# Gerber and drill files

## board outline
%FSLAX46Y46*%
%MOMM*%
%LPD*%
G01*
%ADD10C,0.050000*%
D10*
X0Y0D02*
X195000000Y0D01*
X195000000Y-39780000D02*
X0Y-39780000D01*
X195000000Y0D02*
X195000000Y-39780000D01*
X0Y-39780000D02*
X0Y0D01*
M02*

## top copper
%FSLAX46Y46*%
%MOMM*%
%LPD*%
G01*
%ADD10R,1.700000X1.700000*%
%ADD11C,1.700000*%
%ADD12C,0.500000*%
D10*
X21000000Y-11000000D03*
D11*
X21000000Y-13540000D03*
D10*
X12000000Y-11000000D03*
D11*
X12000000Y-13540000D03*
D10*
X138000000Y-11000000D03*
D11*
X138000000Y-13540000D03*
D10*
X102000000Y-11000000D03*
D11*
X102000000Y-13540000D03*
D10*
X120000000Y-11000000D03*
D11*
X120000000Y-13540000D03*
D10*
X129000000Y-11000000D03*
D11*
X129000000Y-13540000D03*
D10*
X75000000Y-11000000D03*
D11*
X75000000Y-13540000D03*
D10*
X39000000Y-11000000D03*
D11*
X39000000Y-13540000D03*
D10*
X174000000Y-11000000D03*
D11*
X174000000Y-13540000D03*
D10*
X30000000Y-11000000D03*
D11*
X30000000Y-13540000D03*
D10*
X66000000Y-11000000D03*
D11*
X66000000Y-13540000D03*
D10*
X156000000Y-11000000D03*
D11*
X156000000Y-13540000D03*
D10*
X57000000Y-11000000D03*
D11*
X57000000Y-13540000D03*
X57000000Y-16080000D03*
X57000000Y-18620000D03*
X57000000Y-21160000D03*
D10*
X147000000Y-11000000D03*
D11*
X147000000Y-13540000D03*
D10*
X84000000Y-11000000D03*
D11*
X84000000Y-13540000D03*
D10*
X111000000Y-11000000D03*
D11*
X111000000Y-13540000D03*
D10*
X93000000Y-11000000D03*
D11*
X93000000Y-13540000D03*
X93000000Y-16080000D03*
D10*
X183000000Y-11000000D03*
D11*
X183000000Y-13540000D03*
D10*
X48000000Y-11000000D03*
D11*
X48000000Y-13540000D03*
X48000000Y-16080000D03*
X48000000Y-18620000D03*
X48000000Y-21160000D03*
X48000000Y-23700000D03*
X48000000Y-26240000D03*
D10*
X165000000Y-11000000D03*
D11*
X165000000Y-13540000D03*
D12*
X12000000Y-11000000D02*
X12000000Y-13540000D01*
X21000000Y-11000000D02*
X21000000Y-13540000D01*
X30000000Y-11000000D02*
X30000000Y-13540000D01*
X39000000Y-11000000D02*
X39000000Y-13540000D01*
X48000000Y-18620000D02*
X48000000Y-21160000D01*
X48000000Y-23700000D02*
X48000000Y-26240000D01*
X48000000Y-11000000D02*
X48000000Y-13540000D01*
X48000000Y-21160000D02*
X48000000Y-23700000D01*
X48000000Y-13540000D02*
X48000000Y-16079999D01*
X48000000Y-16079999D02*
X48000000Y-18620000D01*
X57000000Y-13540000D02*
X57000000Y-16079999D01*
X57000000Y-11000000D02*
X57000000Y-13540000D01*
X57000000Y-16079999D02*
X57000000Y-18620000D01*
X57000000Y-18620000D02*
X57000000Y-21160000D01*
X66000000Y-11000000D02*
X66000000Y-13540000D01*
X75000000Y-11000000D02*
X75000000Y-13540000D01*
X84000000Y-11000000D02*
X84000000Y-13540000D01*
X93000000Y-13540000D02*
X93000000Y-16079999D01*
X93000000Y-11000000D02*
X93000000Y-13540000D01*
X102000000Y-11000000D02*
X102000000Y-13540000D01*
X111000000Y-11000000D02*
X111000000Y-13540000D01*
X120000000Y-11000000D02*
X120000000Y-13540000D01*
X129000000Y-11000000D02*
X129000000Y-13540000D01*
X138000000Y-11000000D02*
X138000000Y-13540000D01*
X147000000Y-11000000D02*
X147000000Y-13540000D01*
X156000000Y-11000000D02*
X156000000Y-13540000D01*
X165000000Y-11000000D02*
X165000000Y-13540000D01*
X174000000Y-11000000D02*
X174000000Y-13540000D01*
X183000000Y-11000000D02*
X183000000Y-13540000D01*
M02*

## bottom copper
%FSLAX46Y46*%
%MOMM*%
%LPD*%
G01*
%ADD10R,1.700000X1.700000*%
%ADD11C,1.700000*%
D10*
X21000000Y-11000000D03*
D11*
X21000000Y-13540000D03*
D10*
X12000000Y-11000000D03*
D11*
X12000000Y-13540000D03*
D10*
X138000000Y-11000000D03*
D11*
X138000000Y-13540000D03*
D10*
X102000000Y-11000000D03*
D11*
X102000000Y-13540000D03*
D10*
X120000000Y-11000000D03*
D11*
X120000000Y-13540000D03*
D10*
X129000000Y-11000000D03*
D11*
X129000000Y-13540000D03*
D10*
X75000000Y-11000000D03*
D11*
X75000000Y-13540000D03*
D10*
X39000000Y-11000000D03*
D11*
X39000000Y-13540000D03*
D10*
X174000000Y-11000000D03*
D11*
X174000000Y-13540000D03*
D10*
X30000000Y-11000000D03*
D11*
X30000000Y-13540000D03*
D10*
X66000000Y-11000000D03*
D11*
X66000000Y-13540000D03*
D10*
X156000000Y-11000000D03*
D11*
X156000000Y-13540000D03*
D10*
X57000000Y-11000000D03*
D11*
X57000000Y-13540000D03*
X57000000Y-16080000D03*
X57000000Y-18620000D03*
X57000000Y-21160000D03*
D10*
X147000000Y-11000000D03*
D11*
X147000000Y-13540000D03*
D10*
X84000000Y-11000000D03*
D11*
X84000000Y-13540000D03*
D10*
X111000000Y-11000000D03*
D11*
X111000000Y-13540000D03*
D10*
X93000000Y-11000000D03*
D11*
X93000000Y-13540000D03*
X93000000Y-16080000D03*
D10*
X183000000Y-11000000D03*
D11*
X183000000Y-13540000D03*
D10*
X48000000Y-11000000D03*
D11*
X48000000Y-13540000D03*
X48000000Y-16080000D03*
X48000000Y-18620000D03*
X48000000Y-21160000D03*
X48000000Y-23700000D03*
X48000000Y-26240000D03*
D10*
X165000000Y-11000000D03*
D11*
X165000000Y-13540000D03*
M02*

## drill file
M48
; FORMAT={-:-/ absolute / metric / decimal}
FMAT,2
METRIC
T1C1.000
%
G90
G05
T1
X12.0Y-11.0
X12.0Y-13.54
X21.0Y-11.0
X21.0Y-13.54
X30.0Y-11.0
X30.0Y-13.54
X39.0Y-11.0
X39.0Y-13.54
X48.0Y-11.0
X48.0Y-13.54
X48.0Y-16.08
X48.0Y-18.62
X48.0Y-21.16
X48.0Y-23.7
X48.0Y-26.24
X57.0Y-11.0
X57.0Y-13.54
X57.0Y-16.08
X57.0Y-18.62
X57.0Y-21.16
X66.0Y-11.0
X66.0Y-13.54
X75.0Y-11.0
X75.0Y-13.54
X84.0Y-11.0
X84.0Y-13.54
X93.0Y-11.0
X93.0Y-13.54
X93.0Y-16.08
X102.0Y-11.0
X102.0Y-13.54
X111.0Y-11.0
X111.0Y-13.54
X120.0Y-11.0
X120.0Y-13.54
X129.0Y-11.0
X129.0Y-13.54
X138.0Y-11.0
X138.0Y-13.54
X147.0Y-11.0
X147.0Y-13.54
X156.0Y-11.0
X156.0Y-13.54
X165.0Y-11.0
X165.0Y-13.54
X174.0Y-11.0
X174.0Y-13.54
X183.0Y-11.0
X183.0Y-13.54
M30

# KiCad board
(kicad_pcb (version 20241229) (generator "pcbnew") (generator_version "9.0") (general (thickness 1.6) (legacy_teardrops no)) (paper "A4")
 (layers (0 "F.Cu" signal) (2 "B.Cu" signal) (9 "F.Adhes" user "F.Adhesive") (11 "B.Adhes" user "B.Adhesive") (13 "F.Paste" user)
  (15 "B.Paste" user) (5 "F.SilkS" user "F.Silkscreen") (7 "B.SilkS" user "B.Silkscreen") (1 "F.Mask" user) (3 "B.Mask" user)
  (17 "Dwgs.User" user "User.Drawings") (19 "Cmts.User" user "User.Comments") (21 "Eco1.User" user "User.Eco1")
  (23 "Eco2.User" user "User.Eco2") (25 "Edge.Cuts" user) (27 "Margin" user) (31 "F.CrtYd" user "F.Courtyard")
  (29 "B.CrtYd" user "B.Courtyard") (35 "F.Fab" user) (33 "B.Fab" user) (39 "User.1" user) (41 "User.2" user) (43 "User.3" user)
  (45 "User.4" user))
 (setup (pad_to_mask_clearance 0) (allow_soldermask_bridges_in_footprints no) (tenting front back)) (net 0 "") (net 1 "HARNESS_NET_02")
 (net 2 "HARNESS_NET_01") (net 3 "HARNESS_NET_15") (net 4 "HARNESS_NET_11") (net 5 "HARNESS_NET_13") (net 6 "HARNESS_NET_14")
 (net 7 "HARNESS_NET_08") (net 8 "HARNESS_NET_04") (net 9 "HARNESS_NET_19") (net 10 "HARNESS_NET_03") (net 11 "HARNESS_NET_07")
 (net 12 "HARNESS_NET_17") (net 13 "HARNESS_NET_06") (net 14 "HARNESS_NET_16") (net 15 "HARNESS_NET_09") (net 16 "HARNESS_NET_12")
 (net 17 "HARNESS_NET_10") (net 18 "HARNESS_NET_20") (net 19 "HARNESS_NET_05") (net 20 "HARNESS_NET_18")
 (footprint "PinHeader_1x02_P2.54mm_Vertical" (layer "F.Cu") (at 21 11)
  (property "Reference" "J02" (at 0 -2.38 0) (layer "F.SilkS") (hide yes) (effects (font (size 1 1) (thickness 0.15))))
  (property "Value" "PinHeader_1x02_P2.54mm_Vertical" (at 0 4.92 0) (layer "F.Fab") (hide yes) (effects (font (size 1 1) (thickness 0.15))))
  (pad "1" thru_hole rect (at 0 0) (size 1.7 1.7) (drill 1) (layers "*.Cu" "*.Mask") (remove_unused_layers no) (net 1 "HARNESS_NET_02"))
  (pad "2" thru_hole circle (at 0 2.54) (size 1.7 1.7) (drill 1) (layers "*.Cu" "*.Mask") (remove_unused_layers no) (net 1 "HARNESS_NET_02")))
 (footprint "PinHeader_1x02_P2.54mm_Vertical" (layer "F.Cu") (at 12 11)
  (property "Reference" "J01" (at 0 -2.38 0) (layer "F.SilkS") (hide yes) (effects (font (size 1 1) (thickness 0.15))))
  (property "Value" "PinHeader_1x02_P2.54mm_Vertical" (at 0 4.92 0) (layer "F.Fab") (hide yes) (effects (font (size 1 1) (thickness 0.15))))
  (pad "1" thru_hole rect (at 0 0) (size 1.7 1.7) (drill 1) (layers "*.Cu" "*.Mask") (remove_unused_layers no) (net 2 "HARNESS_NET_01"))
  (pad "2" thru_hole circle (at 0 2.54) (size 1.7 1.7) (drill 1) (layers "*.Cu" "*.Mask") (remove_unused_layers no) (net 2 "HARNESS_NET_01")))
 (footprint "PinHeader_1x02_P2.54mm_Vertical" (layer "F.Cu") (at 138 11)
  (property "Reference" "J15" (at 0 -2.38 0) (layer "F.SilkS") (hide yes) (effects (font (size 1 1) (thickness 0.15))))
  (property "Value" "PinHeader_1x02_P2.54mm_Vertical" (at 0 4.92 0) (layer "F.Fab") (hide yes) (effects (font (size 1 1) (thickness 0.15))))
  (pad "1" thru_hole rect (at 0 0) (size 1.7 1.7) (drill 1) (layers "*.Cu" "*.Mask") (remove_unused_layers no) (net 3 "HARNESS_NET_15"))
  (pad "2" thru_hole circle (at 0 2.54) (size 1.7 1.7) (drill 1) (layers "*.Cu" "*.Mask") (remove_unused_layers no) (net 3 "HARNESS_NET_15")))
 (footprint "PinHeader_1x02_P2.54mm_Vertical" (layer "F.Cu") (at 102 11)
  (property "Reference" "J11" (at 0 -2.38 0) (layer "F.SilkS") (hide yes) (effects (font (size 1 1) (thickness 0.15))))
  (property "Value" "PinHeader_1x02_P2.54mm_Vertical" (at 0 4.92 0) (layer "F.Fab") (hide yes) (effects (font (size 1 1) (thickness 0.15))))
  (pad "1" thru_hole rect (at 0 0) (size 1.7 1.7) (drill 1) (layers "*.Cu" "*.Mask") (remove_unused_layers no) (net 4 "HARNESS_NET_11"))
  (pad "2" thru_hole circle (at 0 2.54) (size 1.7 1.7) (drill 1) (layers "*.Cu" "*.Mask") (remove_unused_layers no) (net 4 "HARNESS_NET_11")))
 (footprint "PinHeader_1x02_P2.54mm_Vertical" (layer "F.Cu") (at 120 11)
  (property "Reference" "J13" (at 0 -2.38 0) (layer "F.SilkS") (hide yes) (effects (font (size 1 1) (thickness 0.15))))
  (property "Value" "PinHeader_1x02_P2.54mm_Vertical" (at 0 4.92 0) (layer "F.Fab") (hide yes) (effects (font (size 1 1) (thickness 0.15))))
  (pad "1" thru_hole rect (at 0 0) (size 1.7 1.7) (drill 1) (layers "*.Cu" "*.Mask") (remove_unused_layers no) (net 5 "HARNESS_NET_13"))
  (pad "2" thru_hole circle (at 0 2.54) (size 1.7 1.7) (drill 1) (layers "*.Cu" "*.Mask") (remove_unused_layers no) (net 5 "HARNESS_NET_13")))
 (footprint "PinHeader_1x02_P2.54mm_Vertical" (layer "F.Cu") (at 129 11)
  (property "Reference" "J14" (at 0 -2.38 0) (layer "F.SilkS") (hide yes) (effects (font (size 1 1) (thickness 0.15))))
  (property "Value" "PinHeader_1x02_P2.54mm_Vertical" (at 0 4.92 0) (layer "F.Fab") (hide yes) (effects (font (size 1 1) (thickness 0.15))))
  (pad "1" thru_hole rect (at 0 0) (size 1.7 1.7) (drill 1) (layers "*.Cu" "*.Mask") (remove_unused_layers no) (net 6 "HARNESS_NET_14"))
  (pad "2" thru_hole circle (at 0 2.54) (size 1.7 1.7) (drill 1) (layers "*.Cu" "*.Mask") (remove_unused_layers no) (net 6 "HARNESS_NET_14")))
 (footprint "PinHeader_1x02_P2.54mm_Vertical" (layer "F.Cu") (at 75 11)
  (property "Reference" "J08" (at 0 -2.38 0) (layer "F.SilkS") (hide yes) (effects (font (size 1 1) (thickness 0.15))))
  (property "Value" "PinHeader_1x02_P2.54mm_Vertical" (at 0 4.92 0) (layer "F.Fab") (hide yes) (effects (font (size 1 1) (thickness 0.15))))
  (pad "1" thru_hole rect (at 0 0) (size 1.7 1.7) (drill 1) (layers "*.Cu" "*.Mask") (remove_unused_layers no) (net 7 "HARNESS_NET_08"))
  (pad "2" thru_hole circle (at 0 2.54) (size 1.7 1.7) (drill 1) (layers "*.Cu" "*.Mask") (remove_unused_layers no) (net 7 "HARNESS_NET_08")))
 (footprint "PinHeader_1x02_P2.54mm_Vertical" (layer "F.Cu") (at 39 11)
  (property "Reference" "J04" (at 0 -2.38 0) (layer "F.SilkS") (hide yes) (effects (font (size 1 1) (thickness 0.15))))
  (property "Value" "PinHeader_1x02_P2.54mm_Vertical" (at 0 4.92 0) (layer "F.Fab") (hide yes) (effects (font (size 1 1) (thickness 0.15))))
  (pad "1" thru_hole rect (at 0 0) (size 1.7 1.7) (drill 1) (layers "*.Cu" "*.Mask") (remove_unused_layers no) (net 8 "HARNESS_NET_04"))
  (pad "2" thru_hole circle (at 0 2.54) (size 1.7 1.7) (drill 1) (layers "*.Cu" "*.Mask") (remove_unused_layers no) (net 8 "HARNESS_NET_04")))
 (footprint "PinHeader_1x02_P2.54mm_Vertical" (layer "F.Cu") (at 174 11)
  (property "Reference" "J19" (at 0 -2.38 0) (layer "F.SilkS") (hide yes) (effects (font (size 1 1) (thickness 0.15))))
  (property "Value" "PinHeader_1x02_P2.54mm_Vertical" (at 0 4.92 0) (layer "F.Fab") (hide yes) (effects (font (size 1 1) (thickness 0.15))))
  (pad "1" thru_hole rect (at 0 0) (size 1.7 1.7) (drill 1) (layers "*.Cu" "*.Mask") (remove_unused_layers no) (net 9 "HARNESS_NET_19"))
  (pad "2" thru_hole circle (at 0 2.54) (size 1.7 1.7) (drill 1) (layers "*.Cu" "*.Mask") (remove_unused_layers no) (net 9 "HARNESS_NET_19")))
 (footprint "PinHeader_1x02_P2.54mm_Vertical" (layer "F.Cu") (at 30 11)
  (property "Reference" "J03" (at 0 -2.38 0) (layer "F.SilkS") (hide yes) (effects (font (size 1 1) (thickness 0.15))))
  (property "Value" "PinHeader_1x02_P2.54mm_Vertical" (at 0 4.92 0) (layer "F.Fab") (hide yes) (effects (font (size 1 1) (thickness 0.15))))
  (pad "1" thru_hole rect (at 0 0) (size 1.7 1.7) (drill 1) (layers "*.Cu" "*.Mask") (remove_unused_layers no) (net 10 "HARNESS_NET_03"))
  (pad "2" thru_hole circle (at 0 2.54) (size 1.7 1.7) (drill 1) (layers "*.Cu" "*.Mask") (remove_unused_layers no)
   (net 10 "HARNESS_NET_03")))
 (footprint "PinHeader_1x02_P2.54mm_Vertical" (layer "F.Cu") (at 66 11)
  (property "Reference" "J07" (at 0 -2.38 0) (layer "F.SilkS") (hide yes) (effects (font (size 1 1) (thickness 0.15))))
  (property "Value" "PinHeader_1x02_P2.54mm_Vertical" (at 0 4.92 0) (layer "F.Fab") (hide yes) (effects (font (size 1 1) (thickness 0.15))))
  (pad "1" thru_hole rect (at 0 0) (size 1.7 1.7) (drill 1) (layers "*.Cu" "*.Mask") (remove_unused_layers no) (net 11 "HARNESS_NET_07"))
  (pad "2" thru_hole circle (at 0 2.54) (size 1.7 1.7) (drill 1) (layers "*.Cu" "*.Mask") (remove_unused_layers no)
   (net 11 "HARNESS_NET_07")))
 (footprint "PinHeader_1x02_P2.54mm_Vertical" (layer "F.Cu") (at 156 11)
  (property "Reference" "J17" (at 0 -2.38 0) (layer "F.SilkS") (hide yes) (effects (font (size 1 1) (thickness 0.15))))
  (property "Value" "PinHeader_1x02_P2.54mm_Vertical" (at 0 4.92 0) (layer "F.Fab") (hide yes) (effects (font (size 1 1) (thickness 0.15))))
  (pad "1" thru_hole rect (at 0 0) (size 1.7 1.7) (drill 1) (layers "*.Cu" "*.Mask") (remove_unused_layers no) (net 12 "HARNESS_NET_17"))
  (pad "2" thru_hole circle (at 0 2.54) (size 1.7 1.7) (drill 1) (layers "*.Cu" "*.Mask") (remove_unused_layers no)
   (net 12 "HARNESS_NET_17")))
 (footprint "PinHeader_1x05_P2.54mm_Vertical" (layer "F.Cu") (at 57 11)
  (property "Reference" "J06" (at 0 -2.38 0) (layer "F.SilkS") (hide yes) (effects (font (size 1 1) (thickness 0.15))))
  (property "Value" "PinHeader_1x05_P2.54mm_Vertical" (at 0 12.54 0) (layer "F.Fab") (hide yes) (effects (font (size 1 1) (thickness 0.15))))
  (pad "1" thru_hole rect (at 0 0) (size 1.7 1.7) (drill 1) (layers "*.Cu" "*.Mask") (remove_unused_layers no) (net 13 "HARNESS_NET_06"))
  (pad "2" thru_hole circle (at 0 2.54) (size 1.7 1.7) (drill 1) (layers "*.Cu" "*.Mask") (remove_unused_layers no)
   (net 13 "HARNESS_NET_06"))
  (pad "3" thru_hole circle (at 0 5.08) (size 1.7 1.7) (drill 1) (layers "*.Cu" "*.Mask") (remove_unused_layers no)
   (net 13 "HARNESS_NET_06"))
  (pad "4" thru_hole circle (at 0 7.62) (size 1.7 1.7) (drill 1) (layers "*.Cu" "*.Mask") (remove_unused_layers no)
   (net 13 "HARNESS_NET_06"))
  (pad "5" thru_hole circle (at 0 10.16) (size 1.7 1.7) (drill 1) (layers "*.Cu" "*.Mask") (remove_unused_layers no)
   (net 13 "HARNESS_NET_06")))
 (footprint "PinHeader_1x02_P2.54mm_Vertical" (layer "F.Cu") (at 147 11)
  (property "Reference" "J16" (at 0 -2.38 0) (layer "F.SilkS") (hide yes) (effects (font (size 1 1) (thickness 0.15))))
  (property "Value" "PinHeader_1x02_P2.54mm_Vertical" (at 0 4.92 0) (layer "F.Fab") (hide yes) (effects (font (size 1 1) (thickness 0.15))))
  (pad "1" thru_hole rect (at 0 0) (size 1.7 1.7) (drill 1) (layers "*.Cu" "*.Mask") (remove_unused_layers no) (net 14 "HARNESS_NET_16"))
  (pad "2" thru_hole circle (at 0 2.54) (size 1.7 1.7) (drill 1) (layers "*.Cu" "*.Mask") (remove_unused_layers no)
   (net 14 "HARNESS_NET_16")))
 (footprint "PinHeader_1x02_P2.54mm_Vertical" (layer "F.Cu") (at 84 11)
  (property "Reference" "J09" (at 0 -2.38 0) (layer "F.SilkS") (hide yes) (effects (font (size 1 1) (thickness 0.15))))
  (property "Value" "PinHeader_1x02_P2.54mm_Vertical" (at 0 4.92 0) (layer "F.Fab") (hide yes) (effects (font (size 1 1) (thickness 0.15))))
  (pad "1" thru_hole rect (at 0 0) (size 1.7 1.7) (drill 1) (layers "*.Cu" "*.Mask") (remove_unused_layers no) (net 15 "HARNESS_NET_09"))
  (pad "2" thru_hole circle (at 0 2.54) (size 1.7 1.7) (drill 1) (layers "*.Cu" "*.Mask") (remove_unused_layers no)
   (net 15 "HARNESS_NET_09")))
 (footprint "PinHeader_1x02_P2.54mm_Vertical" (layer "F.Cu") (at 111 11)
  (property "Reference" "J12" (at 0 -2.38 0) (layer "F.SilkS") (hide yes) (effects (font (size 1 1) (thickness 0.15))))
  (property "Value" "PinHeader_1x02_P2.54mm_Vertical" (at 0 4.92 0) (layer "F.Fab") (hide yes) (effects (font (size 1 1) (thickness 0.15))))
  (pad "1" thru_hole rect (at 0 0) (size 1.7 1.7) (drill 1) (layers "*.Cu" "*.Mask") (remove_unused_layers no) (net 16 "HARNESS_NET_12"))
  (pad "2" thru_hole circle (at 0 2.54) (size 1.7 1.7) (drill 1) (layers "*.Cu" "*.Mask") (remove_unused_layers no)
   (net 16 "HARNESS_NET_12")))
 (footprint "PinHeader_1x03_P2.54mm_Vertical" (layer "F.Cu") (at 93 11)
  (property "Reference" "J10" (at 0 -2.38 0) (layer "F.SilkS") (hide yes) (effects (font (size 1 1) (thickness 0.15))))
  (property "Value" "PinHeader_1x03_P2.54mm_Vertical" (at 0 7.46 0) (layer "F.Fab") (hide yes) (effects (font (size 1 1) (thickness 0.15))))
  (pad "1" thru_hole rect (at 0 0) (size 1.7 1.7) (drill 1) (layers "*.Cu" "*.Mask") (remove_unused_layers no) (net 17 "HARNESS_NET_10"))
  (pad "2" thru_hole circle (at 0 2.54) (size 1.7 1.7) (drill 1) (layers "*.Cu" "*.Mask") (remove_unused_layers no)
   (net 17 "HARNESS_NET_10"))
  (pad "3" thru_hole circle (at 0 5.08) (size 1.7 1.7) (drill 1) (layers "*.Cu" "*.Mask") (remove_unused_layers no)
   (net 17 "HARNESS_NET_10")))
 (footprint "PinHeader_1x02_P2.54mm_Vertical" (layer "F.Cu") (at 183 11)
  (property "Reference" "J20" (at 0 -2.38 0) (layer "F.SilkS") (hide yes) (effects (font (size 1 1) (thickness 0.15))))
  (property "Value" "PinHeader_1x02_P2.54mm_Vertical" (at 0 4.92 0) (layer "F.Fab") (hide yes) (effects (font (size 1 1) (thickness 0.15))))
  (pad "1" thru_hole rect (at 0 0) (size 1.7 1.7) (drill 1) (layers "*.Cu" "*.Mask") (remove_unused_layers no) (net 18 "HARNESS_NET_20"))
  (pad "2" thru_hole circle (at 0 2.54) (size 1.7 1.7) (drill 1) (layers "*.Cu" "*.Mask") (remove_unused_layers no)
   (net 18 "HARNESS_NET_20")))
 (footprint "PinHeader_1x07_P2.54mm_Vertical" (layer "F.Cu") (at 48 11)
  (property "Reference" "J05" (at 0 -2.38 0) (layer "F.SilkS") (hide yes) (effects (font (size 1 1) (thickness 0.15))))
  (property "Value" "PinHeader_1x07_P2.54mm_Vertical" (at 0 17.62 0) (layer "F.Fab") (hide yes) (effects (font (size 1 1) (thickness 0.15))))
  (pad "1" thru_hole rect (at 0 0) (size 1.7 1.7) (drill 1) (layers "*.Cu" "*.Mask") (remove_unused_layers no) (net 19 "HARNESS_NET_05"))
  (pad "2" thru_hole circle (at 0 2.54) (size 1.7 1.7) (drill 1) (layers "*.Cu" "*.Mask") (remove_unused_layers no)
   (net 19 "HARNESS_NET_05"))
  (pad "3" thru_hole circle (at 0 5.08) (size 1.7 1.7) (drill 1) (layers "*.Cu" "*.Mask") (remove_unused_layers no)
   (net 19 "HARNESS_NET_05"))
  (pad "4" thru_hole circle (at 0 7.62) (size 1.7 1.7) (drill 1) (layers "*.Cu" "*.Mask") (remove_unused_layers no)
   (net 19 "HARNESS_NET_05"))
  (pad "5" thru_hole circle (at 0 10.16) (size 1.7 1.7) (drill 1) (layers "*.Cu" "*.Mask") (remove_unused_layers no)
   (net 19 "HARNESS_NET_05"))
  (pad "6" thru_hole circle (at 0 12.7) (size 1.7 1.7) (drill 1) (layers "*.Cu" "*.Mask") (remove_unused_layers no)
   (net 19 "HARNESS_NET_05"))
  (pad "7" thru_hole circle (at 0 15.24) (size 1.7 1.7) (drill 1) (layers "*.Cu" "*.Mask") (remove_unused_layers no)
   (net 19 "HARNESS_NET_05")))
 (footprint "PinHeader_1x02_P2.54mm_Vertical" (layer "F.Cu") (at 165 11)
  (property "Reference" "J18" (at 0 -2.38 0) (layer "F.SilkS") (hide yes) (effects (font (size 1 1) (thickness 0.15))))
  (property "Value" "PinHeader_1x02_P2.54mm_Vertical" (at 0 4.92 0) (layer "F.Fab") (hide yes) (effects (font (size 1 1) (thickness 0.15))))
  (pad "1" thru_hole rect (at 0 0) (size 1.7 1.7) (drill 1) (layers "*.Cu" "*.Mask") (remove_unused_layers no) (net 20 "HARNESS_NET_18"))
  (pad "2" thru_hole circle (at 0 2.54) (size 1.7 1.7) (drill 1) (layers "*.Cu" "*.Mask") (remove_unused_layers no)
   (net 20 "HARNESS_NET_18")))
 (gr_line (start 0 0) (end 195 0) (stroke (width 0.05) (type default)) (layer "Edge.Cuts"))
 (gr_line (start 195 39.78) (end 0 39.78) (stroke (width 0.05) (type default)) (layer "Edge.Cuts"))
 (gr_line (start 195 0) (end 195 39.78) (stroke (width 0.05) (type default)) (layer "Edge.Cuts"))
 (gr_line (start 0 39.78) (end 0 0) (stroke (width 0.05) (type default)) (layer "Edge.Cuts"))
 (segment (start 12 11) (end 12 13.54) (width 0.5) (layer "F.Cu") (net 2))
 (segment (start 21 11) (end 21 13.54) (width 0.5) (layer "F.Cu") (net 1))
 (segment (start 30 11) (end 30 13.54) (width 0.5) (layer "F.Cu") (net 10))
 (segment (start 39 11) (end 39 13.54) (width 0.5) (layer "F.Cu") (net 8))
 (segment (start 48 18.62) (end 48 21.16) (width 0.5) (layer "F.Cu") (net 19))
 (segment (start 48 23.7) (end 48 26.24) (width 0.5) (layer "F.Cu") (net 19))
 (segment (start 48 11) (end 48 13.54) (width 0.5) (layer "F.Cu") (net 19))
 (segment (start 48 21.16) (end 48 23.7) (width 0.5) (layer "F.Cu") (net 19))
 (segment (start 48 13.54) (end 48 16.079999) (width 0.5) (layer "F.Cu") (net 19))
 (segment (start 48 16.079999) (end 48 18.62) (width 0.5) (layer "F.Cu") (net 19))
 (segment (start 57 13.54) (end 57 16.079999) (width 0.5) (layer "F.Cu") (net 13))
 (segment (start 57 11) (end 57 13.54) (width 0.5) (layer "F.Cu") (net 13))
 (segment (start 57 16.079999) (end 57 18.62) (width 0.5) (layer "F.Cu") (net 13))
 (segment (start 57 18.62) (end 57 21.16) (width 0.5) (layer "F.Cu") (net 13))
 (segment (start 66 11) (end 66 13.54) (width 0.5) (layer "F.Cu") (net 11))
 (segment (start 75 11) (end 75 13.54) (width 0.5) (layer "F.Cu") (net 7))
 (segment (start 84 11) (end 84 13.54) (width 0.5) (layer "F.Cu") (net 15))
 (segment (start 93 13.54) (end 93 16.079999) (width 0.5) (layer "F.Cu") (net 17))
 (segment (start 93 11) (end 93 13.54) (width 0.5) (layer "F.Cu") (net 17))
 (segment (start 102 11) (end 102 13.54) (width 0.5) (layer "F.Cu") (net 4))
 (segment (start 111 11) (end 111 13.54) (width 0.5) (layer "F.Cu") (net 16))
 (segment (start 120 11) (end 120 13.54) (width 0.5) (layer "F.Cu") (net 5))
 (segment (start 129 11) (end 129 13.54) (width 0.5) (layer "F.Cu") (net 6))
 (segment (start 138 11) (end 138 13.54) (width 0.5) (layer "F.Cu") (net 3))
 (segment (start 147 11) (end 147 13.54) (width 0.5) (layer "F.Cu") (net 14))
 (segment (start 156 11) (end 156 13.54) (width 0.5) (layer "F.Cu") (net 12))
 (segment (start 165 11) (end 165 13.54) (width 0.5) (layer "F.Cu") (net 20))
 (segment (start 174 11) (end 174 13.54) (width 0.5) (layer "F.Cu") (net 9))
 (segment (start 183 11) (end 183 13.54) (width 0.5) (layer "F.Cu") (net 18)))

